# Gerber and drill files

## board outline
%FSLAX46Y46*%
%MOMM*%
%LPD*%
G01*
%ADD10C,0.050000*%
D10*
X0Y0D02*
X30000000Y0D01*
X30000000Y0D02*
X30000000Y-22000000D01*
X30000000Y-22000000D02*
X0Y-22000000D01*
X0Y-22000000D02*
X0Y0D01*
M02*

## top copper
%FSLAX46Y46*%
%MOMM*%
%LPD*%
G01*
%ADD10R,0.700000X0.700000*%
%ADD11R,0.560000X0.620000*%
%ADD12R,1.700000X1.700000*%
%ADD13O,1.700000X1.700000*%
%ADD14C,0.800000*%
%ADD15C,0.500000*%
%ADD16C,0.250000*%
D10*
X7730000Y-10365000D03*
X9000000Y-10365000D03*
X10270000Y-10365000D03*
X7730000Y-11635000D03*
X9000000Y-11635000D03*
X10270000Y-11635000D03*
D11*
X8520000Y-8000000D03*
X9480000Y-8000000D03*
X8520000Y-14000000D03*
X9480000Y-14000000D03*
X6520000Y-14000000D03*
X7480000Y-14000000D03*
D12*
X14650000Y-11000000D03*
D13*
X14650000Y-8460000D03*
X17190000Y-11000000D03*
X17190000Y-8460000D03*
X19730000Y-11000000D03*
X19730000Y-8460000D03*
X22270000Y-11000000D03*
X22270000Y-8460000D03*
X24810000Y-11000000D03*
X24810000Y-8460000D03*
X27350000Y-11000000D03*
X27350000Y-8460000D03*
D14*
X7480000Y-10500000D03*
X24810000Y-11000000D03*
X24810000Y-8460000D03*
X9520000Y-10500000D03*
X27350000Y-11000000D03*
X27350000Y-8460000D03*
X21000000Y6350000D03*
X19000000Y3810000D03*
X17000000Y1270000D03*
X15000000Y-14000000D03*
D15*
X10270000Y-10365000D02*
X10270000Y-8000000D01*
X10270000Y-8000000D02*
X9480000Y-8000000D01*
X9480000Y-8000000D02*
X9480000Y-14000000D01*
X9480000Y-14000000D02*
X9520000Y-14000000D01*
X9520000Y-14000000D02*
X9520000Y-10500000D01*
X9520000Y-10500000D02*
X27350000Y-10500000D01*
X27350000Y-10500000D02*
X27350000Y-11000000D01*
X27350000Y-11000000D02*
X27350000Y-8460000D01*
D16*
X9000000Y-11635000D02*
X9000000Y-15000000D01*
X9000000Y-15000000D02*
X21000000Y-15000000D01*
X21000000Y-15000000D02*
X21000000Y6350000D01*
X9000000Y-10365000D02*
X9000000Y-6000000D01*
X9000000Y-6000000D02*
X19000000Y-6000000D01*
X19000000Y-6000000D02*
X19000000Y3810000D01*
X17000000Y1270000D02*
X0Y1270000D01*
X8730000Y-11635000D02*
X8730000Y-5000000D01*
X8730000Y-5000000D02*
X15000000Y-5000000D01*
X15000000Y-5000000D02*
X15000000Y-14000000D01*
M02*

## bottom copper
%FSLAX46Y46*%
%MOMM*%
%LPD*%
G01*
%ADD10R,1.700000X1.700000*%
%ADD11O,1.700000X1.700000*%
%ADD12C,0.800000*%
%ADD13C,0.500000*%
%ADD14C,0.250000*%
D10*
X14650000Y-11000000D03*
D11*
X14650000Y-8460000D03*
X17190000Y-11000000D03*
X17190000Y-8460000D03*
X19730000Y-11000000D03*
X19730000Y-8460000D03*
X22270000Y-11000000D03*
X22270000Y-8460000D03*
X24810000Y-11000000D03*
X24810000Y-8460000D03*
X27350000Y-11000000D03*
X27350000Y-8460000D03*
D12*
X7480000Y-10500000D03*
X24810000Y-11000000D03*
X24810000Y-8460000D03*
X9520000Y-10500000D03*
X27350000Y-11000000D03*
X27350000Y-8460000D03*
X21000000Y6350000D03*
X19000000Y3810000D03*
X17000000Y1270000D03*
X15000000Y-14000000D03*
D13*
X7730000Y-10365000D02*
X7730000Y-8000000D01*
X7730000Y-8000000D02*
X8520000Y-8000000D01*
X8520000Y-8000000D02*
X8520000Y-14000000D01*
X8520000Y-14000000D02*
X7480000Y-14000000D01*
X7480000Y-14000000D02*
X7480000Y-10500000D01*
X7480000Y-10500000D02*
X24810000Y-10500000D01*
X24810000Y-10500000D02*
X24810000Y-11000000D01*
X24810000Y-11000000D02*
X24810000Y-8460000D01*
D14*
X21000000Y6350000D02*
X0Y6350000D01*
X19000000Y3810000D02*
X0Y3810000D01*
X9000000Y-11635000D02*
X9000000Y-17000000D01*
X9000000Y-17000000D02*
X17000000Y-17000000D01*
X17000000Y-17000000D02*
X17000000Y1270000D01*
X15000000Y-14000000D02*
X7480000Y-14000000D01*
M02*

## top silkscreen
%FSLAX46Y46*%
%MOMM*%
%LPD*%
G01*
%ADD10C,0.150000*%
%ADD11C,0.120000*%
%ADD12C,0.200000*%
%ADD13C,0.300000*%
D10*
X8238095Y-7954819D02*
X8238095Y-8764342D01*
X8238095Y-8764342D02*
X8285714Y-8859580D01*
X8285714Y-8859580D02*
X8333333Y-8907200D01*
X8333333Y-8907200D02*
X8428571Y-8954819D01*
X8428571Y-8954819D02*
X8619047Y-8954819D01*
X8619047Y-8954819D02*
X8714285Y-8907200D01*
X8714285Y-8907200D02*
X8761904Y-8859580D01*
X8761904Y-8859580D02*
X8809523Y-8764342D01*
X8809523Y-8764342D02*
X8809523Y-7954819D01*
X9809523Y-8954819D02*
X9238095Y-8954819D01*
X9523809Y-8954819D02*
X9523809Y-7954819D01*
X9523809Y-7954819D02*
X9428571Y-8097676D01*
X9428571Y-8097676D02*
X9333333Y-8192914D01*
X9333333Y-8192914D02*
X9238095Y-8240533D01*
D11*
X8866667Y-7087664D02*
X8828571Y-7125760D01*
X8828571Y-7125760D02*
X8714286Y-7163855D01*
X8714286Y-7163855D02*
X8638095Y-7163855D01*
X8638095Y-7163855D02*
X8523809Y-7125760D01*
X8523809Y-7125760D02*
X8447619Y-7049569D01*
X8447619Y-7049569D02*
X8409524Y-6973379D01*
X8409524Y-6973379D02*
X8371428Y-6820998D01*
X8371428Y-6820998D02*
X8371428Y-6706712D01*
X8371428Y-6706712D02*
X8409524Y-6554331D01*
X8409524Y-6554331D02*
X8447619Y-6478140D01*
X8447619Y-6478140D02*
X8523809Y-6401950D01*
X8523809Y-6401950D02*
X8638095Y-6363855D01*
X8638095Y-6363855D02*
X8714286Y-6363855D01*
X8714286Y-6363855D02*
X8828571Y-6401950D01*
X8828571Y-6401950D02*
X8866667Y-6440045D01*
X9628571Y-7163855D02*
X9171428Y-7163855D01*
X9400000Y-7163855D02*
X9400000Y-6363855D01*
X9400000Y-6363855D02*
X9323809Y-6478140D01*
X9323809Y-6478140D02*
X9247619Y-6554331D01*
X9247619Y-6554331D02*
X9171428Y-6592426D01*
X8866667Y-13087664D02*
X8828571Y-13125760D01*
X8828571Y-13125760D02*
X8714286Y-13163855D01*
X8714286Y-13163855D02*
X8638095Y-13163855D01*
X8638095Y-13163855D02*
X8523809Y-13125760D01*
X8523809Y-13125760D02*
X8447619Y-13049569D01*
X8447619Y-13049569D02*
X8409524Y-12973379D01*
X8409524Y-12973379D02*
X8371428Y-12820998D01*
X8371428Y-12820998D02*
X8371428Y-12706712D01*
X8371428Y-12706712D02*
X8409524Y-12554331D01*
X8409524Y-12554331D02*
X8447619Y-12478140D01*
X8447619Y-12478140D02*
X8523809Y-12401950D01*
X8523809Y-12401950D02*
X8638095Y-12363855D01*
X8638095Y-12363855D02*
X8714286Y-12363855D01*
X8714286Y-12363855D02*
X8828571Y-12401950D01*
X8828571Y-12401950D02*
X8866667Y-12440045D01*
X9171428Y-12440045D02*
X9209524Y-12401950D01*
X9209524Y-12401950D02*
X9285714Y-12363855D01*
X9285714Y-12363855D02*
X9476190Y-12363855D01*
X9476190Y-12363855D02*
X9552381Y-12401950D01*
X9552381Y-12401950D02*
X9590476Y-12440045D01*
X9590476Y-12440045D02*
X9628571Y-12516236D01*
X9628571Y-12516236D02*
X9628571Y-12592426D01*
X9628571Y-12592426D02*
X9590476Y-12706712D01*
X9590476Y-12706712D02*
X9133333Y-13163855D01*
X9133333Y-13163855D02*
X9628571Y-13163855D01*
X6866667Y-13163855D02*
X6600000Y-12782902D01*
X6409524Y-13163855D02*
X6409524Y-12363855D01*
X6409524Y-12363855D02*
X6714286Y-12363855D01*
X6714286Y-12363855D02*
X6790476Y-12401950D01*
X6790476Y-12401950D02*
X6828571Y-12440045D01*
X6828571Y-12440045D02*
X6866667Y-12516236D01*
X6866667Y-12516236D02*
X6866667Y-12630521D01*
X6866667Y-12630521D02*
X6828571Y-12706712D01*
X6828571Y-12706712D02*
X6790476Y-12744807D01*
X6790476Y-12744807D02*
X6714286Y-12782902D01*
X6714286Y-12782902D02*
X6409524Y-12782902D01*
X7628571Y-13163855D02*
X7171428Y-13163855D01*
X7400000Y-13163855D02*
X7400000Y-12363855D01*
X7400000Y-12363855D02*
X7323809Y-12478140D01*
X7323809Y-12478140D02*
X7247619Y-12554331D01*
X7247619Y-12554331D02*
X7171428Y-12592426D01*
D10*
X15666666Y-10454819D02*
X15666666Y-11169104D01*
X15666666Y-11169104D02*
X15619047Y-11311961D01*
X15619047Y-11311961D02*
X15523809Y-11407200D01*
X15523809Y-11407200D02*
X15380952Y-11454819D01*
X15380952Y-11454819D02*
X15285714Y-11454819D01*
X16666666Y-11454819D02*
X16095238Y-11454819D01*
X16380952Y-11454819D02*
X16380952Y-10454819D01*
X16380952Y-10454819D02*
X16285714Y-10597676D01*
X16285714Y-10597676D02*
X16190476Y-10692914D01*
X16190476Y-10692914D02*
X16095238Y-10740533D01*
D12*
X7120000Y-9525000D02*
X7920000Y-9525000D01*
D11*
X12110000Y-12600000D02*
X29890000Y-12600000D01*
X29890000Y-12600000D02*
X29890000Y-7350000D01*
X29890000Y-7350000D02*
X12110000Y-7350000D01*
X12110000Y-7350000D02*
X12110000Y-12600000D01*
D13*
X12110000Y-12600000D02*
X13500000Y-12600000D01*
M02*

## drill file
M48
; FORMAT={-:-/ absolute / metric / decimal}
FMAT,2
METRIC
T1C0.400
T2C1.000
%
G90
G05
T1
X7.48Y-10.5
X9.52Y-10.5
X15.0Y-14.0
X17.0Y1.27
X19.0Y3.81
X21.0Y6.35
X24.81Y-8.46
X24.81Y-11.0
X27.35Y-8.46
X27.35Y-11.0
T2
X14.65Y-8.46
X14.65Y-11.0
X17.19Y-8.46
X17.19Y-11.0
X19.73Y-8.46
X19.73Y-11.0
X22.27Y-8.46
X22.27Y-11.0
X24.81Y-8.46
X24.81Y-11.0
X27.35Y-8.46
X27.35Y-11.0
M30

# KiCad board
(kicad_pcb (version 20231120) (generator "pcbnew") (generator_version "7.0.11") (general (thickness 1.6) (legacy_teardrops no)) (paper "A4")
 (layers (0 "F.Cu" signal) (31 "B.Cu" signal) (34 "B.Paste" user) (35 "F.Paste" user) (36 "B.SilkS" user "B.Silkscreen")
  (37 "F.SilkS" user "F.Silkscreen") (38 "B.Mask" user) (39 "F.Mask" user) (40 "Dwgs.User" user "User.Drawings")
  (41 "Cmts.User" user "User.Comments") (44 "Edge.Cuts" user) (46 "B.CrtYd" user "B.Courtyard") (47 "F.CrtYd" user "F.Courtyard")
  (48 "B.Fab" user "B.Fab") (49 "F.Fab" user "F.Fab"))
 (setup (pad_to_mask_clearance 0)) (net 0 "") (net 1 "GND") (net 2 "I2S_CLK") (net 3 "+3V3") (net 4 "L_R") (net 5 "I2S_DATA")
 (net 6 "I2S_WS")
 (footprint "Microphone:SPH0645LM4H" (layer "F.Cu") (at 9 11)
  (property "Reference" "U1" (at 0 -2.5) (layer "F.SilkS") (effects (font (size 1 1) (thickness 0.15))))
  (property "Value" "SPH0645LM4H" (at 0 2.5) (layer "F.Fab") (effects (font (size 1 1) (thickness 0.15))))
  (fp_line (start -1.88 -1.475) (end -1.08 -1.475) (layer "F.SilkS") (width 0.2))
  (pad "1" smd rect (at -1.27 -0.635) (size 0.7 0.7) (layers "F.Cu" "F.Paste" "F.Mask") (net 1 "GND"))
  (pad "2" smd rect (at 0 -0.635) (size 0.7 0.7) (layers "F.Cu" "F.Paste" "F.Mask") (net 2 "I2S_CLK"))
  (pad "3" smd rect (at 1.27 -0.635) (size 0.7 0.7) (layers "F.Cu" "F.Paste" "F.Mask") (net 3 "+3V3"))
  (pad "4" smd rect (at -1.27 0.635) (size 0.7 0.7) (layers "F.Cu" "F.Paste" "F.Mask") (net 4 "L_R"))
  (pad "5" smd rect (at 0 0.635) (size 0.7 0.7) (layers "F.Cu" "F.Paste" "F.Mask") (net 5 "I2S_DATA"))
  (pad "6" smd rect (at 1.27 0.635) (size 0.7 0.7) (layers "F.Cu" "F.Paste" "F.Mask") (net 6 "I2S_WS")))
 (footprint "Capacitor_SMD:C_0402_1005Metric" (layer "F.Cu") (at 9 8)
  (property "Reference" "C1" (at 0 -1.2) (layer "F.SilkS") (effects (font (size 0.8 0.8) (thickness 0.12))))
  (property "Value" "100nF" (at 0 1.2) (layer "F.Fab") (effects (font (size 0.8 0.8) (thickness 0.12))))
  (pad "1" smd rect (at -0.48 0) (size 0.56 0.62) (layers "F.Cu" "F.Paste" "F.Mask") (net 3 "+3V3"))
  (pad "2" smd rect (at 0.48 0) (size 0.56 0.62) (layers "F.Cu" "F.Paste" "F.Mask") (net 1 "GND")))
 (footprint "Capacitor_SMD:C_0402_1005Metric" (layer "F.Cu") (at 9 14)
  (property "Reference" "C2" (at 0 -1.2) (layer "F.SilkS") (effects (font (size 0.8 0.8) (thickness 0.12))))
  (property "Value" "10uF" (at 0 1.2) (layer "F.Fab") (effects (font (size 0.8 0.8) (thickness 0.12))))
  (pad "1" smd rect (at -0.48 0) (size 0.56 0.62) (layers "F.Cu" "F.Paste" "F.Mask") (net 3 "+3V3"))
  (pad "2" smd rect (at 0.48 0) (size 0.56 0.62) (layers "F.Cu" "F.Paste" "F.Mask") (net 1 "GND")))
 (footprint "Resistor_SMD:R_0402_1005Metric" (layer "F.Cu") (at 7 14)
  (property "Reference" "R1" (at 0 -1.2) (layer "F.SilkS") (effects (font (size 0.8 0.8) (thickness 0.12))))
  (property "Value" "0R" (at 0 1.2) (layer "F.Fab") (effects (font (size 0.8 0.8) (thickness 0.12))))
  (pad "1" smd rect (at -0.48 0) (size 0.56 0.62) (layers "F.Cu" "F.Paste" "F.Mask") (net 4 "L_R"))
  (pad "2" smd rect (at 0.48 0) (size 0.56 0.62) (layers "F.Cu" "F.Paste" "F.Mask") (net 1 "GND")))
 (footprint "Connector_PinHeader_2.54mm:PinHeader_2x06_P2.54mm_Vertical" (layer "F.Cu") (at 21 11 90)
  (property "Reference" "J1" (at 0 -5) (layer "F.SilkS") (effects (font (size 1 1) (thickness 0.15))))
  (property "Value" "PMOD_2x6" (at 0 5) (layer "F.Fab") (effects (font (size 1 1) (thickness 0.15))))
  (fp_line (start -1.6 -8.89) (end -1.6 8.89) (layer "F.SilkS") (width 0.12))
  (fp_line (start -1.6 8.89) (end 3.65 8.89) (layer "F.SilkS") (width 0.12))
  (fp_line (start 3.65 8.89) (end 3.65 -8.89) (layer "F.SilkS") (width 0.12))
  (fp_line (start 3.65 -8.89) (end -1.6 -8.89) (layer "F.SilkS") (width 0.12))
  (fp_line (start -1.6 -8.89) (end -1.6 -7.5) (layer "F.SilkS") (width 0.3))
  (pad "1" thru_hole rect (at 0 -6.35) (size 1.7 1.7) (drill 1.0) (layers "*.Cu" "*.Mask") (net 5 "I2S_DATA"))
  (pad "2" thru_hole oval (at 2.54 -6.35) (size 1.7 1.7) (drill 1.0) (layers "*.Cu" "*.Mask"))
  (pad "3" thru_hole oval (at 0 -3.81) (size 1.7 1.7) (drill 1.0) (layers "*.Cu" "*.Mask") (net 2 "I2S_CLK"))
  (pad "4" thru_hole oval (at 2.54 -3.81) (size 1.7 1.7) (drill 1.0) (layers "*.Cu" "*.Mask"))
  (pad "5" thru_hole oval (at 0 -1.27) (size 1.7 1.7) (drill 1.0) (layers "*.Cu" "*.Mask") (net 6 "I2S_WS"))
  (pad "6" thru_hole oval (at 2.54 -1.27) (size 1.7 1.7) (drill 1.0) (layers "*.Cu" "*.Mask"))
  (pad "7" thru_hole oval (at 0 1.27) (size 1.7 1.7) (drill 1.0) (layers "*.Cu" "*.Mask"))
  (pad "8" thru_hole oval (at 2.54 1.27) (size 1.7 1.7) (drill 1.0) (layers "*.Cu" "*.Mask"))
  (pad "9" thru_hole oval (at 0 3.81) (size 1.7 1.7) (drill 1.0) (layers "*.Cu" "*.Mask") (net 1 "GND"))
  (pad "10" thru_hole oval (at 2.54 3.81) (size 1.7 1.7) (drill 1.0) (layers "*.Cu" "*.Mask") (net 1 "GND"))
  (pad "11" thru_hole oval (at 0 6.35) (size 1.7 1.7) (drill 1.0) (layers "*.Cu" "*.Mask") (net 3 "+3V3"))
  (pad "12" thru_hole oval (at 2.54 6.35) (size 1.7 1.7) (drill 1.0) (layers "*.Cu" "*.Mask") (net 3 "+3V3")))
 (gr_line (start 0 0) (end 30 0) (layer "Edge.Cuts") (width 0.05))
 (gr_line (start 30 0) (end 30 22) (layer "Edge.Cuts") (width 0.05))
 (gr_line (start 30 22) (end 0 22) (layer "Edge.Cuts") (width 0.05))
 (gr_line (start 0 22) (end 0 0) (layer "Edge.Cuts") (width 0.05))
 (segment (start 7.73 10.365) (end 7.73 8) (width 0.5) (layer "B.Cu") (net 1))
 (segment (start 7.73 8) (end 8.52 8) (width 0.5) (layer "B.Cu") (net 1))
 (segment (start 8.52 8) (end 8.52 14) (width 0.5) (layer "B.Cu") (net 1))
 (segment (start 8.52 14) (end 7.48 14) (width 0.5) (layer "B.Cu") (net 1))
 (segment (start 7.48 14) (end 7.48 10.5) (width 0.5) (layer "B.Cu") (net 1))
 (via (at 7.48 10.5) (size 0.8) (drill 0.4) (layers "F.Cu" "B.Cu") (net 1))
 (segment (start 7.48 10.5) (end 24.81 10.5) (width 0.5) (layer "B.Cu") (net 1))
 (segment (start 24.81 10.5) (end 24.81 11) (width 0.5) (layer "B.Cu") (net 1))
 (via (at 24.81 11) (size 0.8) (drill 0.4) (layers "F.Cu" "B.Cu") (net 1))
 (segment (start 24.81 11) (end 24.81 8.46) (width 0.5) (layer "B.Cu") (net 1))
 (via (at 24.81 8.46) (size 0.8) (drill 0.4) (layers "F.Cu" "B.Cu") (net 1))
 (segment (start 10.27 10.365) (end 10.27 8) (width 0.5) (layer "F.Cu") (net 3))
 (segment (start 10.27 8) (end 9.48 8) (width 0.5) (layer "F.Cu") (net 3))
 (segment (start 9.48 8) (end 9.48 14) (width 0.5) (layer "F.Cu") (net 3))
 (segment (start 9.48 14) (end 9.52 14) (width 0.5) (layer "F.Cu") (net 3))
 (segment (start 9.52 14) (end 9.52 10.5) (width 0.5) (layer "F.Cu") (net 3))
 (via (at 9.52 10.5) (size 0.8) (drill 0.4) (layers "F.Cu" "B.Cu") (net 3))
 (segment (start 9.52 10.5) (end 27.35 10.5) (width 0.5) (layer "F.Cu") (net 3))
 (segment (start 27.35 10.5) (end 27.35 11) (width 0.5) (layer "F.Cu") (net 3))
 (via (at 27.35 11) (size 0.8) (drill 0.4) (layers "F.Cu" "B.Cu") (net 3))
 (segment (start 27.35 11) (end 27.35 8.46) (width 0.5) (layer "F.Cu") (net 3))
 (via (at 27.35 8.46) (size 0.8) (drill 0.4) (layers "F.Cu" "B.Cu") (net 3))
 (segment (start 9 11.635) (end 9 15) (width 0.25) (layer "F.Cu") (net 5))
 (segment (start 9 15) (end 21 15) (width 0.25) (layer "F.Cu") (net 5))
 (segment (start 21 15) (end 21 -6.35) (width 0.25) (layer "F.Cu") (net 5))
 (via (at 21 -6.35) (size 0.8) (drill 0.4) (layers "F.Cu" "B.Cu") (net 5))
 (segment (start 21 -6.35) (end 0 -6.35) (width 0.25) (layer "B.Cu") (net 5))
 (segment (start 9 10.365) (end 9 6) (width 0.25) (layer "F.Cu") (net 2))
 (segment (start 9 6) (end 19 6) (width 0.25) (layer "F.Cu") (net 2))
 (segment (start 19 6) (end 19 -3.81) (width 0.25) (layer "F.Cu") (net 2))
 (via (at 19 -3.81) (size 0.8) (drill 0.4) (layers "F.Cu" "B.Cu") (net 2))
 (segment (start 19 -3.81) (end 0 -3.81) (width 0.25) (layer "B.Cu") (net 2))
 (segment (start 9 11.635) (end 9 17) (width 0.25) (layer "B.Cu") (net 6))
 (segment (start 9 17) (end 17 17) (width 0.25) (layer "B.Cu") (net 6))
 (segment (start 17 17) (end 17 -1.27) (width 0.25) (layer "B.Cu") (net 6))
 (via (at 17 -1.27) (size 0.8) (drill 0.4) (layers "F.Cu" "B.Cu") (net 6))
 (segment (start 17 -1.27) (end 0 -1.27) (width 0.25) (layer "F.Cu") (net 6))
 (segment (start 8.73 11.635) (end 8.73 5) (width 0.25) (layer "F.Cu") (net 4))
 (segment (start 8.73 5) (end 15 5) (width 0.25) (layer "F.Cu") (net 4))
 (segment (start 15 5) (end 15 14) (width 0.25) (layer "F.Cu") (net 4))
 (via (at 15 14) (size 0.8) (drill 0.4) (layers "F.Cu" "B.Cu") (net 4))
 (segment (start 15 14) (end 7.48 14) (width 0.25) (layer "B.Cu") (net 4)))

